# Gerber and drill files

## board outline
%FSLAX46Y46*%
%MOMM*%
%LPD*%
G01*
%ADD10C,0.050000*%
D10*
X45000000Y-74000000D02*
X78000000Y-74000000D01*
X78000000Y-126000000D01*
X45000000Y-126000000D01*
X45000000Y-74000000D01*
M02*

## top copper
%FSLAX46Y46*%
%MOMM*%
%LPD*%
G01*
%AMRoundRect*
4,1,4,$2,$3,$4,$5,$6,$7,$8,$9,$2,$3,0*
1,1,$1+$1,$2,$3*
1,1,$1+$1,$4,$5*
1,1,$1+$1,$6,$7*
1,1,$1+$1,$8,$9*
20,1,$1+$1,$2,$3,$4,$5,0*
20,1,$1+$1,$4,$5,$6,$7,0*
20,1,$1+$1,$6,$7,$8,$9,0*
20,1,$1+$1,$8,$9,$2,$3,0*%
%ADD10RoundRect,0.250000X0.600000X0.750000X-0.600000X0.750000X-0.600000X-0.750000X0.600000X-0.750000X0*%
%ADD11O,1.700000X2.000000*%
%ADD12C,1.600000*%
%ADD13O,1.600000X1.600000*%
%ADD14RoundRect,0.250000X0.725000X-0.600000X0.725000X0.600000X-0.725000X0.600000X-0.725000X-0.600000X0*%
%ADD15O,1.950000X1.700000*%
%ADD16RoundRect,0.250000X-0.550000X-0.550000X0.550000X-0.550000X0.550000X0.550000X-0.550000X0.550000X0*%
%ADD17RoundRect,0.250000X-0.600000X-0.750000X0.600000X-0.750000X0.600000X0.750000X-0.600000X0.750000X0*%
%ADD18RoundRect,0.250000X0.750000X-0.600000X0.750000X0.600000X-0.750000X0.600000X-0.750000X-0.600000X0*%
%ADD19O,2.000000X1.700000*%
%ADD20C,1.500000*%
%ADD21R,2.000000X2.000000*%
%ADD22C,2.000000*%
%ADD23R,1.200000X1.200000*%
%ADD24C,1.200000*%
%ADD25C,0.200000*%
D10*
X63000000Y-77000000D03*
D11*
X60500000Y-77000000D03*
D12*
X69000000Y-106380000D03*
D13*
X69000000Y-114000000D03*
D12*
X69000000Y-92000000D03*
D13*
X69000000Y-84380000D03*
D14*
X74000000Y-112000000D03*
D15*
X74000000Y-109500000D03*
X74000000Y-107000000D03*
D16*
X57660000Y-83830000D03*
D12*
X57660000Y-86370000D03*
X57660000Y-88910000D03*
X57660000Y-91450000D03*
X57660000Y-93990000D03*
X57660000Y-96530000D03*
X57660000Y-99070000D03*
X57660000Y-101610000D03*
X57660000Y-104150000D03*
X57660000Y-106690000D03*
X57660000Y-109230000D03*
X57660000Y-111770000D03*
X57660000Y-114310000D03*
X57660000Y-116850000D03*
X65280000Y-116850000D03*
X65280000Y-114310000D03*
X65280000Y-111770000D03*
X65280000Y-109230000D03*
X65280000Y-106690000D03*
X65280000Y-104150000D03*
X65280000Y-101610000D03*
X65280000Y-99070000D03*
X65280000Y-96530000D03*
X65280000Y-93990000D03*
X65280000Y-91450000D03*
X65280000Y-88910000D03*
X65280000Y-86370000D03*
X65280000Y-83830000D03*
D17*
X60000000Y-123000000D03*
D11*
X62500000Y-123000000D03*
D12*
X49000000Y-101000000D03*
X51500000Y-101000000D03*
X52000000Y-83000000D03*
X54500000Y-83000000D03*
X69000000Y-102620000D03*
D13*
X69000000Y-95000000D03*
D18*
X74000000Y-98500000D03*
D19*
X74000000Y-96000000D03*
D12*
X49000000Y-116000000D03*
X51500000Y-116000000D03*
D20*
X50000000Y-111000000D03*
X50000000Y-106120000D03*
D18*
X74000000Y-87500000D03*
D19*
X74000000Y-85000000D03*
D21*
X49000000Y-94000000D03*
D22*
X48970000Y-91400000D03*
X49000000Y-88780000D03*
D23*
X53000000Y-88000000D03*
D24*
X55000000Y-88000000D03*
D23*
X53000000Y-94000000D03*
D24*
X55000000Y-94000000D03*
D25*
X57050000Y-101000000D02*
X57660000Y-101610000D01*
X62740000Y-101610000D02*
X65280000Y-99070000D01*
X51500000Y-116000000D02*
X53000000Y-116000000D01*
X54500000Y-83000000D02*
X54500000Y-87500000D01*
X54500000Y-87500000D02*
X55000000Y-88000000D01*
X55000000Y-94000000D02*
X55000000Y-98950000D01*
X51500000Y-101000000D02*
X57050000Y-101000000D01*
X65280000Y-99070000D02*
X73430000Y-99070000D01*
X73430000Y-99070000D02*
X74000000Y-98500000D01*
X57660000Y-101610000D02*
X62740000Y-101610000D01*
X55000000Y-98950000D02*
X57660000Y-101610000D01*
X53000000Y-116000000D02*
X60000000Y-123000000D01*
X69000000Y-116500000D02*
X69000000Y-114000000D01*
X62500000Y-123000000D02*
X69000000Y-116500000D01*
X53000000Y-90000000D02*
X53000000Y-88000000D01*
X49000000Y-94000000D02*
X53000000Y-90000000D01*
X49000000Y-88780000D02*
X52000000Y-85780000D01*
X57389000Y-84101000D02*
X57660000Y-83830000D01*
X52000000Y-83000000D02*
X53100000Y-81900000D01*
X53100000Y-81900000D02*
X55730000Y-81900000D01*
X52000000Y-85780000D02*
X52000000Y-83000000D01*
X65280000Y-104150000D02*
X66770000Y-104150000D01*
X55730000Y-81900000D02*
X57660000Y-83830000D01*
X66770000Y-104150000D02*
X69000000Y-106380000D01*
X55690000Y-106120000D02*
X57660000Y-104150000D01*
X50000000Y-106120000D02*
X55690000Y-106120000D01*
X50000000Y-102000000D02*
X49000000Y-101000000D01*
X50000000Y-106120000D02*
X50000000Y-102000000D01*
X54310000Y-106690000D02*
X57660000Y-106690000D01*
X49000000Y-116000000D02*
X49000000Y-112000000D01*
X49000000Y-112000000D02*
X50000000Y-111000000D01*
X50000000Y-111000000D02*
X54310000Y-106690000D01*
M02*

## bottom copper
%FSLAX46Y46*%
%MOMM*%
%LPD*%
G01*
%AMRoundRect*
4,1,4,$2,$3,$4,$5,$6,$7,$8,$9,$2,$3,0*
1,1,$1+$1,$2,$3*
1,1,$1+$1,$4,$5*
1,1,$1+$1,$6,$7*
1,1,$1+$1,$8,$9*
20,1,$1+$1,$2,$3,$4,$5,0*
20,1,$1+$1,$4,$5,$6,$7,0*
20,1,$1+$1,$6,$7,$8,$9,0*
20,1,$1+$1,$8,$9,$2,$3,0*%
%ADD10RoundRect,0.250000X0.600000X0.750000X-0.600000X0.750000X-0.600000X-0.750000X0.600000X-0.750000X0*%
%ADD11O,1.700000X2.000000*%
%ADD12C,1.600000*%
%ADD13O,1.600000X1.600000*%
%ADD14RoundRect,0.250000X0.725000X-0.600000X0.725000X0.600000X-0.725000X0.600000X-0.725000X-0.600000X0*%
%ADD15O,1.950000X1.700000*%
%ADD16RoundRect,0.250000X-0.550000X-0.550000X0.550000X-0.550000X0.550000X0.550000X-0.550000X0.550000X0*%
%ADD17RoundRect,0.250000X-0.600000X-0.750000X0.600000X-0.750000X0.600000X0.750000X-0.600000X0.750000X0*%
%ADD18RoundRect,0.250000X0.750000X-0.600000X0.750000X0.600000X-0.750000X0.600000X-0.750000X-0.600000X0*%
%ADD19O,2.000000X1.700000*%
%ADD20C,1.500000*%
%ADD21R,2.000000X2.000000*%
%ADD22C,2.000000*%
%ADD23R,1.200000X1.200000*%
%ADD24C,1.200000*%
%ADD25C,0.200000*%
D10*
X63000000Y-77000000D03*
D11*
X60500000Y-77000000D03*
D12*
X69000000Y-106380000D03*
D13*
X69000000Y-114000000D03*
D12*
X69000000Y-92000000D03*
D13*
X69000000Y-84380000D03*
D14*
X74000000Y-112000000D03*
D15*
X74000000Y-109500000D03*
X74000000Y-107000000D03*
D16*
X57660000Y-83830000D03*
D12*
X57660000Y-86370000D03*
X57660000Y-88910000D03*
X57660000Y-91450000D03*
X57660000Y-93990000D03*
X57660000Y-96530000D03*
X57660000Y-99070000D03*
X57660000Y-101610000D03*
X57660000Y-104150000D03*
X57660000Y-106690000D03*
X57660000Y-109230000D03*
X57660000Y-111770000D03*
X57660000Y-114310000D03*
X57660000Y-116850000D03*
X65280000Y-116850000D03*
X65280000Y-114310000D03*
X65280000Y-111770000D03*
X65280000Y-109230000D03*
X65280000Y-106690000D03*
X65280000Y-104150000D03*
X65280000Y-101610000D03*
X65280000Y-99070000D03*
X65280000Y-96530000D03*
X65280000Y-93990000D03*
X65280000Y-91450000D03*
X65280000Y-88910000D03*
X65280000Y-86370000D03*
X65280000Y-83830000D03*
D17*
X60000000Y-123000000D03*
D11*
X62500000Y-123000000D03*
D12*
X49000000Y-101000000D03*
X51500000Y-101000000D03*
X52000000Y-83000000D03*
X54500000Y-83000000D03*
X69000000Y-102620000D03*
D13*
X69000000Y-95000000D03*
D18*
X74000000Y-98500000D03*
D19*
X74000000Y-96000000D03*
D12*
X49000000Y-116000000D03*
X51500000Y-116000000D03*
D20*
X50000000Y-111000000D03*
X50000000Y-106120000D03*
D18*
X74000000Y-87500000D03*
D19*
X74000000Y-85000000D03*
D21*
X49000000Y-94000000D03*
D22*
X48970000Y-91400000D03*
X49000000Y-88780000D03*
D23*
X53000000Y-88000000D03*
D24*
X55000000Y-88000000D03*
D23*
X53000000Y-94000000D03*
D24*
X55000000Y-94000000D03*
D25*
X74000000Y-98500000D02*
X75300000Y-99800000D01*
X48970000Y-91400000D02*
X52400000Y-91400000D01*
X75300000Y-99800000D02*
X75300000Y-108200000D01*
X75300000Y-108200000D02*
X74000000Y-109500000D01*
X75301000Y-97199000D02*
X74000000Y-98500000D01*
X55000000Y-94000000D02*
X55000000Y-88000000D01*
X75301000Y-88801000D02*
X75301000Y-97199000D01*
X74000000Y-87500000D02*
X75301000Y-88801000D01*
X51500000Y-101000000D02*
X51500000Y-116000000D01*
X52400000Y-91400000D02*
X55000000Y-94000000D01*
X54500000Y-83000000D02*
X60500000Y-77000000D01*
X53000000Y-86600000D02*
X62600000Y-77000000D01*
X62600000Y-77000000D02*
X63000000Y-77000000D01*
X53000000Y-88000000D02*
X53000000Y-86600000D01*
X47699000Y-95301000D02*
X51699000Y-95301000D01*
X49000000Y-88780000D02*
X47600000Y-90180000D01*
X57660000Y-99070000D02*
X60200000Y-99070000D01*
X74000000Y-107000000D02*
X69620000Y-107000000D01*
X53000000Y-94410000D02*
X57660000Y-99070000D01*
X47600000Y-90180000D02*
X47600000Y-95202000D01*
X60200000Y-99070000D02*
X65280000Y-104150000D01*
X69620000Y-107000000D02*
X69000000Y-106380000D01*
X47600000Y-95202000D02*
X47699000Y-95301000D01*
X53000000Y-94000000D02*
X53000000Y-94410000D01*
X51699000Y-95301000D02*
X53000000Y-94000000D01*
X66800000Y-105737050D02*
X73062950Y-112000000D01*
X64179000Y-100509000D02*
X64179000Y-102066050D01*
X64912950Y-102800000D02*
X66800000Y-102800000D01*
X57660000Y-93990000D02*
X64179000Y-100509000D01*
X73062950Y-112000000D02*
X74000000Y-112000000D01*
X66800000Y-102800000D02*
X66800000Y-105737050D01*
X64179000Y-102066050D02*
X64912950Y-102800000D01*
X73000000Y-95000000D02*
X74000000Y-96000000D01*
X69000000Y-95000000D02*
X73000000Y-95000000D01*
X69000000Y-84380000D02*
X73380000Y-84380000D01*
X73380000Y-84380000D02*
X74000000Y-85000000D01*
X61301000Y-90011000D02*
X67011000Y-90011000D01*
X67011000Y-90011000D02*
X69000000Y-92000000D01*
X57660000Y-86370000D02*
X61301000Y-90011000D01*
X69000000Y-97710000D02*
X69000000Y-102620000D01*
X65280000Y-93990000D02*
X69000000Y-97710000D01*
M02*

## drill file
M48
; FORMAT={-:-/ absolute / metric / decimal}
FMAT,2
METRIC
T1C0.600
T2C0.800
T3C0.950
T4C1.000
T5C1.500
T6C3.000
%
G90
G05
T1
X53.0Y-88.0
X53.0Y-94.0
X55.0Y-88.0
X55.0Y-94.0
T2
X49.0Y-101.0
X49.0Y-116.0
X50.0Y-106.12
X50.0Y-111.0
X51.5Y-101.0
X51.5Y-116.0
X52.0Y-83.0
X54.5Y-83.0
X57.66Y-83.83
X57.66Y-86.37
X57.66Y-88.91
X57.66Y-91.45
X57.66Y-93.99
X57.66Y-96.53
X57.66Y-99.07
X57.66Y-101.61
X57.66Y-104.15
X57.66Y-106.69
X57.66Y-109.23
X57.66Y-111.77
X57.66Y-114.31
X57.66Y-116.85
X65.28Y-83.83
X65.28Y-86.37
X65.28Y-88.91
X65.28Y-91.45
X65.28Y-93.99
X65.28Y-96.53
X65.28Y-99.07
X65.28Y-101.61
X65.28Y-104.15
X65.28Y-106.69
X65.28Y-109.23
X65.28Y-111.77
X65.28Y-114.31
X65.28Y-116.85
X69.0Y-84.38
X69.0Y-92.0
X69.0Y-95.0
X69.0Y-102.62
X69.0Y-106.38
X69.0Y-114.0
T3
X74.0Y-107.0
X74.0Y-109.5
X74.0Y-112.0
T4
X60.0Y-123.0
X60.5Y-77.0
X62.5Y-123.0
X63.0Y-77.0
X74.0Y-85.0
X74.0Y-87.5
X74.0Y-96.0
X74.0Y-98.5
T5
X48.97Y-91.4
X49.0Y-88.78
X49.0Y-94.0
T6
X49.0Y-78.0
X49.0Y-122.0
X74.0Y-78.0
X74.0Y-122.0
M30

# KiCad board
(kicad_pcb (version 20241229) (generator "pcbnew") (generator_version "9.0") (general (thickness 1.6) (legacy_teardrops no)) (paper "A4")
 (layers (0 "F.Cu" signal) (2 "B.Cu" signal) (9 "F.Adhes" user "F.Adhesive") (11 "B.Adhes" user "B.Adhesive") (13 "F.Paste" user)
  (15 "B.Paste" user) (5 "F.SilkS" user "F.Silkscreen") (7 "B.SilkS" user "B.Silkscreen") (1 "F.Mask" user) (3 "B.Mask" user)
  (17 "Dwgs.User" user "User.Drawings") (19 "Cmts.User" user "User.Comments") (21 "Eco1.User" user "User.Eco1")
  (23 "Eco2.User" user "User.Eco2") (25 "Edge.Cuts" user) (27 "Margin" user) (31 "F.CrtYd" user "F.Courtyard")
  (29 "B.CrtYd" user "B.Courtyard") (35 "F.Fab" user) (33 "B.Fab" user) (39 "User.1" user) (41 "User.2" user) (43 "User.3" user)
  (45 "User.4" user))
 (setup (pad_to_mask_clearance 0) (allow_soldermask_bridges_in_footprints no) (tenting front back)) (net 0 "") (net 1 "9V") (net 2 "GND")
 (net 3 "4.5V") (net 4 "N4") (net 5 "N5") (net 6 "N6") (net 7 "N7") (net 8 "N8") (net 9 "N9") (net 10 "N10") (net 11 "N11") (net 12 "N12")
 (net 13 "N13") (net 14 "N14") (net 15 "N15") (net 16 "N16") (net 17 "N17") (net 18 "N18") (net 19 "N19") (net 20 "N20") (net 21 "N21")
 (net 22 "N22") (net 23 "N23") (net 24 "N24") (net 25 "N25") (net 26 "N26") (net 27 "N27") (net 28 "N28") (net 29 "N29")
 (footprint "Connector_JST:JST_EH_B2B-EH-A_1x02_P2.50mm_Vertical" (layer "F.Cu") (at 63 77 180)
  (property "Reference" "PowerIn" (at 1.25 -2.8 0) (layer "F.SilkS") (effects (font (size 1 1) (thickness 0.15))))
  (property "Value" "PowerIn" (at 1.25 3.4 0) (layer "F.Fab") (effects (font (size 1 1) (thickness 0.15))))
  (pad "1" thru_hole roundrect (at 0 0 180) (size 1.7 2) (drill 1) (layers "*.Cu" "*.Mask") (remove_unused_layers no)
   (roundrect_rratio 0.147059) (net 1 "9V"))
  (pad "2" thru_hole oval (at 2.5 0 180) (size 1.7 2) (drill 1) (layers "*.Cu" "*.Mask") (remove_unused_layers no) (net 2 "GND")))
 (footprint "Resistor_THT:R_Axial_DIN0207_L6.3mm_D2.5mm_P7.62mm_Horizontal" (layer "F.Cu") (at 69 106.38 -90)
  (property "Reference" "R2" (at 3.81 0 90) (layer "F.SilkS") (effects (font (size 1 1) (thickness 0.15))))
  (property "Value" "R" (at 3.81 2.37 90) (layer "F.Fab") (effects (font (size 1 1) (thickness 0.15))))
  (pad "1" thru_hole circle (at 0 0 270) (size 1.6 1.6) (drill 0.8) (layers "*.Cu" "*.Mask") (remove_unused_layers no) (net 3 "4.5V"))
  (pad "2" thru_hole oval (at 7.62 0 270) (size 1.6 1.6) (drill 0.8) (layers "*.Cu" "*.Mask") (remove_unused_layers no) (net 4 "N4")))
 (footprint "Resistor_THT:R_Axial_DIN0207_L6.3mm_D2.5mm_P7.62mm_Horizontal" (layer "F.Cu") (at 69 92 90)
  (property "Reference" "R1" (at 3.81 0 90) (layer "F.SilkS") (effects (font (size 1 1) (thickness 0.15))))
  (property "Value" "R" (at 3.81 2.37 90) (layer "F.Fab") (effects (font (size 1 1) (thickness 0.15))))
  (pad "1" thru_hole circle (at 0 0 90) (size 1.6 1.6) (drill 0.8) (layers "*.Cu" "*.Mask") (remove_unused_layers no) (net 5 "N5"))
  (pad "2" thru_hole oval (at 7.62 0 90) (size 1.6 1.6) (drill 0.8) (layers "*.Cu" "*.Mask") (remove_unused_layers no) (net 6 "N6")))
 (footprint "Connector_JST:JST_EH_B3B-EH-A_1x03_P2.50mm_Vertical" (layer "F.Cu") (at 74 112 90)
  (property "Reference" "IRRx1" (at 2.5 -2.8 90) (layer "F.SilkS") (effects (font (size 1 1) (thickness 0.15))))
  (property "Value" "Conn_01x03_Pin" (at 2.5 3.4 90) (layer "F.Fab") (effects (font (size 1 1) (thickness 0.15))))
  (pad "1" thru_hole roundrect (at 0 0 90) (size 1.7 1.95) (drill 0.95) (layers "*.Cu" "*.Mask") (remove_unused_layers no)
   (roundrect_rratio 0.147059) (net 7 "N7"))
  (pad "2" thru_hole oval (at 2.5 0 90) (size 1.7 1.95) (drill 0.95) (layers "*.Cu" "*.Mask") (remove_unused_layers no) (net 2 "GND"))
  (pad "3" thru_hole oval (at 5 0 90) (size 1.7 1.95) (drill 0.95) (layers "*.Cu" "*.Mask") (remove_unused_layers no) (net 3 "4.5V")))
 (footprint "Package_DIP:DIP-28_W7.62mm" (layer "F.Cu") (at 57.66 83.83)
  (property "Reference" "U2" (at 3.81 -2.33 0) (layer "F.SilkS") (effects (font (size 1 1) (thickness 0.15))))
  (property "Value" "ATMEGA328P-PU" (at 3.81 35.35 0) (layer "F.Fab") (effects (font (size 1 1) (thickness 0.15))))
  (pad "1" thru_hole roundrect (at 0 0) (size 1.6 1.6) (drill 0.8) (layers "*.Cu" "*.Mask") (remove_unused_layers no)
   (roundrect_rratio 0.15625) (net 3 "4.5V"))
  (pad "2" thru_hole circle (at 0 2.54) (size 1.6 1.6) (drill 0.8) (layers "*.Cu" "*.Mask") (remove_unused_layers no) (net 5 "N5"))
  (pad "3" thru_hole circle (at 0 5.08) (size 1.6 1.6) (drill 0.8) (layers "*.Cu" "*.Mask") (remove_unused_layers no) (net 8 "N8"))
  (pad "4" thru_hole circle (at 0 7.62) (size 1.6 1.6) (drill 0.8) (layers "*.Cu" "*.Mask") (remove_unused_layers no) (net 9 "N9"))
  (pad "5" thru_hole circle (at 0 10.16) (size 1.6 1.6) (drill 0.8) (layers "*.Cu" "*.Mask") (remove_unused_layers no) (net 7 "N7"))
  (pad "6" thru_hole circle (at 0 12.7) (size 1.6 1.6) (drill 0.8) (layers "*.Cu" "*.Mask") (remove_unused_layers no) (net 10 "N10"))
  (pad "7" thru_hole circle (at 0 15.24) (size 1.6 1.6) (drill 0.8) (layers "*.Cu" "*.Mask") (remove_unused_layers no) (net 3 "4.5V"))
  (pad "8" thru_hole circle (at 0 17.78) (size 1.6 1.6) (drill 0.8) (layers "*.Cu" "*.Mask") (remove_unused_layers no) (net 2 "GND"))
  (pad "9" thru_hole circle (at 0 20.32) (size 1.6 1.6) (drill 0.8) (layers "*.Cu" "*.Mask") (remove_unused_layers no) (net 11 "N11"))
  (pad "10" thru_hole circle (at 0 22.86) (size 1.6 1.6) (drill 0.8) (layers "*.Cu" "*.Mask") (remove_unused_layers no) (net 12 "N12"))
  (pad "11" thru_hole circle (at 0 25.4) (size 1.6 1.6) (drill 0.8) (layers "*.Cu" "*.Mask") (remove_unused_layers no) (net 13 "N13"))
  (pad "12" thru_hole circle (at 0 27.94) (size 1.6 1.6) (drill 0.8) (layers "*.Cu" "*.Mask") (remove_unused_layers no) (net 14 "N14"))
  (pad "13" thru_hole circle (at 0 30.48) (size 1.6 1.6) (drill 0.8) (layers "*.Cu" "*.Mask") (remove_unused_layers no) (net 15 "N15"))
  (pad "14" thru_hole circle (at 0 33.02) (size 1.6 1.6) (drill 0.8) (layers "*.Cu" "*.Mask") (remove_unused_layers no) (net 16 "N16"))
  (pad "15" thru_hole circle (at 7.62 33.02) (size 1.6 1.6) (drill 0.8) (layers "*.Cu" "*.Mask") (remove_unused_layers no) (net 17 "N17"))
  (pad "16" thru_hole circle (at 7.62 30.48) (size 1.6 1.6) (drill 0.8) (layers "*.Cu" "*.Mask") (remove_unused_layers no) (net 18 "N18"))
  (pad "17" thru_hole circle (at 7.62 27.94) (size 1.6 1.6) (drill 0.8) (layers "*.Cu" "*.Mask") (remove_unused_layers no) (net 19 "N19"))
  (pad "18" thru_hole circle (at 7.62 25.4) (size 1.6 1.6) (drill 0.8) (layers "*.Cu" "*.Mask") (remove_unused_layers no) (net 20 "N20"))
  (pad "19" thru_hole circle (at 7.62 22.86) (size 1.6 1.6) (drill 0.8) (layers "*.Cu" "*.Mask") (remove_unused_layers no) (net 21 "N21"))
  (pad "20" thru_hole circle (at 7.62 20.32) (size 1.6 1.6) (drill 0.8) (layers "*.Cu" "*.Mask") (remove_unused_layers no) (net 3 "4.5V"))
  (pad "21" thru_hole circle (at 7.62 17.78) (size 1.6 1.6) (drill 0.8) (layers "*.Cu" "*.Mask") (remove_unused_layers no) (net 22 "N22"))
  (pad "22" thru_hole circle (at 7.62 15.24) (size 1.6 1.6) (drill 0.8) (layers "*.Cu" "*.Mask") (remove_unused_layers no) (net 2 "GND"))
  (pad "23" thru_hole circle (at 7.62 12.7) (size 1.6 1.6) (drill 0.8) (layers "*.Cu" "*.Mask") (remove_unused_layers no) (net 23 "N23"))
  (pad "24" thru_hole circle (at 7.62 10.16) (size 1.6 1.6) (drill 0.8) (layers "*.Cu" "*.Mask") (remove_unused_layers no) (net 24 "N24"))
  (pad "25" thru_hole circle (at 7.62 7.62) (size 1.6 1.6) (drill 0.8) (layers "*.Cu" "*.Mask") (remove_unused_layers no) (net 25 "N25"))
  (pad "26" thru_hole circle (at 7.62 5.08) (size 1.6 1.6) (drill 0.8) (layers "*.Cu" "*.Mask") (remove_unused_layers no) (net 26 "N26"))
  (pad "27" thru_hole circle (at 7.62 2.54) (size 1.6 1.6) (drill 0.8) (layers "*.Cu" "*.Mask") (remove_unused_layers no) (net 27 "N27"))
  (pad "28" thru_hole circle (at 7.62 0) (size 1.6 1.6) (drill 0.8) (layers "*.Cu" "*.Mask") (remove_unused_layers no) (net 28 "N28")))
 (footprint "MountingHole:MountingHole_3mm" (layer "F.Cu") (at 49 122)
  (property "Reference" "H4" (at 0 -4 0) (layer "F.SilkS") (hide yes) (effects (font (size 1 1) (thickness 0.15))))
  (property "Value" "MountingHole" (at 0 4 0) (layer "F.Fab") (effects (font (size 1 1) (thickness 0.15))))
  (pad "" np_thru_hole circle (at 0 0) (size 3 3) (drill 3) (layers "*.Cu" "*.Mask")))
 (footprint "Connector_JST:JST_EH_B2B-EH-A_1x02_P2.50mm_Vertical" (layer "F.Cu") (at 60 123)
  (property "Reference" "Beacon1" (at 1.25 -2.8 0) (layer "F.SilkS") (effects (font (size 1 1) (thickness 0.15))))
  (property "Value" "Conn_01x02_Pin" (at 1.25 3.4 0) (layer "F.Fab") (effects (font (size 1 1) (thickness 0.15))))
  (pad "1" thru_hole roundrect (at 0 0) (size 1.7 2) (drill 1) (layers "*.Cu" "*.Mask") (remove_unused_layers no)
   (roundrect_rratio 0.147059) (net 2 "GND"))
  (pad "2" thru_hole oval (at 2.5 0) (size 1.7 2) (drill 1) (layers "*.Cu" "*.Mask") (remove_unused_layers no) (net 4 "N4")))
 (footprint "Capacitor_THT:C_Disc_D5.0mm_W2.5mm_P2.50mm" (layer "F.Cu") (at 49 101)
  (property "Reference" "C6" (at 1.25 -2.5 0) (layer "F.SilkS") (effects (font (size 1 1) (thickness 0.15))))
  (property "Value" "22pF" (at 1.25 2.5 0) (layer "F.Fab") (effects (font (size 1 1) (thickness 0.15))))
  (pad "1" thru_hole circle (at 0 0) (size 1.6 1.6) (drill 0.8) (layers "*.Cu" "*.Mask") (remove_unused_layers no) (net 11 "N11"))
  (pad "2" thru_hole circle (at 2.5 0) (size 1.6 1.6) (drill 0.8) (layers "*.Cu" "*.Mask") (remove_unused_layers no) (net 2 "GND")))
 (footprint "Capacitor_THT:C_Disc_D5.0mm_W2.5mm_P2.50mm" (layer "F.Cu") (at 52 83)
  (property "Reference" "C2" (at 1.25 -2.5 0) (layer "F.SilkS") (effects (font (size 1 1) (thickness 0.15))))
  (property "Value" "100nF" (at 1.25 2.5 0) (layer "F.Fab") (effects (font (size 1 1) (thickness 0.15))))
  (pad "1" thru_hole circle (at 0 0) (size 1.6 1.6) (drill 0.8) (layers "*.Cu" "*.Mask") (remove_unused_layers no) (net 3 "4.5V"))
  (pad "2" thru_hole circle (at 2.5 0) (size 1.6 1.6) (drill 0.8) (layers "*.Cu" "*.Mask") (remove_unused_layers no) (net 2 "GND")))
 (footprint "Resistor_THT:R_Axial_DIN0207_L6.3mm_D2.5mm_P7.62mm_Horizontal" (layer "F.Cu") (at 69 102.62 90)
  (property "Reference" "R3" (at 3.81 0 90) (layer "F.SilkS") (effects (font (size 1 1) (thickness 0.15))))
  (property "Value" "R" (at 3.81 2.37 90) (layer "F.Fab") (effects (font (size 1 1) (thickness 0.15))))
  (pad "1" thru_hole circle (at 0 0 90) (size 1.6 1.6) (drill 0.8) (layers "*.Cu" "*.Mask") (remove_unused_layers no) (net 24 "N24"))
  (pad "2" thru_hole oval (at 7.62 0 90) (size 1.6 1.6) (drill 0.8) (layers "*.Cu" "*.Mask") (remove_unused_layers no) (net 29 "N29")))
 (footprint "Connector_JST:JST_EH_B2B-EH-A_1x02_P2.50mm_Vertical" (layer "F.Cu") (at 74 98.5 90)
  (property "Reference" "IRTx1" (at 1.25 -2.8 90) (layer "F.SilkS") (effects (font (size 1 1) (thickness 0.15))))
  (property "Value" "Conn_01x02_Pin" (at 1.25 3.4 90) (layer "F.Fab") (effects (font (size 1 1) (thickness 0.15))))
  (pad "1" thru_hole roundrect (at 0 0 90) (size 1.7 2) (drill 1) (layers "*.Cu" "*.Mask") (remove_unused_layers no)
   (roundrect_rratio 0.147059) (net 2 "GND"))
  (pad "2" thru_hole oval (at 2.5 0 90) (size 1.7 2) (drill 1) (layers "*.Cu" "*.Mask") (remove_unused_layers no) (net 29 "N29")))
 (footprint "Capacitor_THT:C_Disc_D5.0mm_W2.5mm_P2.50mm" (layer "F.Cu") (at 49 116)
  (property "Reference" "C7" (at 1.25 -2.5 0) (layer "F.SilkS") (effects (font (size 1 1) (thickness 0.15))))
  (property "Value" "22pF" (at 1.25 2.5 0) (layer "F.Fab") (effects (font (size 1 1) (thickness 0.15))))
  (pad "1" thru_hole circle (at 0 0) (size 1.6 1.6) (drill 0.8) (layers "*.Cu" "*.Mask") (remove_unused_layers no) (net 12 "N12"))
  (pad "2" thru_hole circle (at 2.5 0) (size 1.6 1.6) (drill 0.8) (layers "*.Cu" "*.Mask") (remove_unused_layers no) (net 2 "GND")))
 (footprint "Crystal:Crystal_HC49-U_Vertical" (layer "F.Cu") (at 50 111 90)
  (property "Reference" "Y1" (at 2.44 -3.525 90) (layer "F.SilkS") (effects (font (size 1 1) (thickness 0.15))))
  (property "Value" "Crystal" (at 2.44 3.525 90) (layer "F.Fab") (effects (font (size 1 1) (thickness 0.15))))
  (pad "1" thru_hole circle (at 0 0 90) (size 1.5 1.5) (drill 0.8) (layers "*.Cu" "*.Mask") (remove_unused_layers no) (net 12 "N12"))
  (pad "2" thru_hole circle (at 4.88 0 90) (size 1.5 1.5) (drill 0.8) (layers "*.Cu" "*.Mask") (remove_unused_layers no) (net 11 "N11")))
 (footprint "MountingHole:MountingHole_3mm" (layer "F.Cu") (at 74 122)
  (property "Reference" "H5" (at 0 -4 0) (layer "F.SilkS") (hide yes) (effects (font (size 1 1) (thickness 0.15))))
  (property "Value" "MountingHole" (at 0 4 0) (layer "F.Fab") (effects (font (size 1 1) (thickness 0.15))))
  (pad "" np_thru_hole circle (at 0 0) (size 3 3) (drill 3) (layers "*.Cu" "*.Mask")))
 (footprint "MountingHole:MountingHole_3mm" (layer "F.Cu") (at 49 78)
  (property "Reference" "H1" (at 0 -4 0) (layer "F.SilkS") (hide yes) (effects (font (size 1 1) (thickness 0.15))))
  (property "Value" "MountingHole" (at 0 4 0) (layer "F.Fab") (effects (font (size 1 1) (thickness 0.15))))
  (pad "" np_thru_hole circle (at 0 0) (size 3 3) (drill 3) (layers "*.Cu" "*.Mask")))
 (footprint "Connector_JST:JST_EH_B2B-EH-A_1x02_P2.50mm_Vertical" (layer "F.Cu") (at 74 87.5 90)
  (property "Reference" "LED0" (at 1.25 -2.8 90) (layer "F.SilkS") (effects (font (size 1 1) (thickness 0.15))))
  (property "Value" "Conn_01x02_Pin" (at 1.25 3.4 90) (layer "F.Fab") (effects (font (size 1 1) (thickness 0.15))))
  (pad "1" thru_hole roundrect (at 0 0 90) (size 1.7 2) (drill 1) (layers "*.Cu" "*.Mask") (remove_unused_layers no)
   (roundrect_rratio 0.147059) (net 2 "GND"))
  (pad "2" thru_hole oval (at 2.5 0 90) (size 1.7 2) (drill 1) (layers "*.Cu" "*.Mask") (remove_unused_layers no) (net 6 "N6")))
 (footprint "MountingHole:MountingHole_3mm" (layer "F.Cu") (at 74 78)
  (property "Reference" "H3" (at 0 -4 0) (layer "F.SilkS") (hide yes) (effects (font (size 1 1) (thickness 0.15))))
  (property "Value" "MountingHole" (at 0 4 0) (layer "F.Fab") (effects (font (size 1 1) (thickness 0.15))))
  (pad "" np_thru_hole circle (at 0 0) (size 3 3) (drill 3) (layers "*.Cu" "*.Mask")))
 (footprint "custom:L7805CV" (layer "F.Cu") (at 48.08 95.01 90)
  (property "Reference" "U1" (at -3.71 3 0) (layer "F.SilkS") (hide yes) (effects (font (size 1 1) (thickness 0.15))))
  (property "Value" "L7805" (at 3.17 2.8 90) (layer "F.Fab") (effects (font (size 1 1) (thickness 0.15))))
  (pad "1" thru_hole rect (at 1.01 0.92 90) (size 2 2) (drill 1.5) (layers "*.Cu" "*.Mask") (remove_unused_layers no) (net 1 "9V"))
  (pad "2" thru_hole circle (at 3.61 0.89 90) (size 2 2) (drill 1.5) (layers "*.Cu" "*.Mask") (remove_unused_layers no) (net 2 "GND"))
  (pad "3" thru_hole circle (at 6.23 0.92 90) (size 2 2) (drill 1.5) (layers "*.Cu" "*.Mask") (remove_unused_layers no) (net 3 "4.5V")))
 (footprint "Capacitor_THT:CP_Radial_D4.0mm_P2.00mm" (layer "F.Cu") (at 53 88)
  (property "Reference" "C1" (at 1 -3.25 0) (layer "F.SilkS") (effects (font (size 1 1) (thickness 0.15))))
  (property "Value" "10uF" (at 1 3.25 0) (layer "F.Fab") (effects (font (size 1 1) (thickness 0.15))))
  (pad "1" thru_hole rect (at 0 0) (size 1.2 1.2) (drill 0.6) (layers "*.Cu" "*.Mask") (remove_unused_layers no) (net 1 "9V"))
  (pad "2" thru_hole circle (at 2 0) (size 1.2 1.2) (drill 0.6) (layers "*.Cu" "*.Mask") (remove_unused_layers no) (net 2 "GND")))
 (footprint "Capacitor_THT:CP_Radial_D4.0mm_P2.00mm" (layer "F.Cu") (at 53 94)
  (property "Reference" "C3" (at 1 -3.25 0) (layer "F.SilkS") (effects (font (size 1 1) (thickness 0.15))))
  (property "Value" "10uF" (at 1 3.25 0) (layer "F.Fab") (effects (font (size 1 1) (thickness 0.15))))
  (pad "1" thru_hole rect (at 0 0) (size 1.2 1.2) (drill 0.6) (layers "*.Cu" "*.Mask") (remove_unused_layers no) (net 3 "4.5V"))
  (pad "2" thru_hole circle (at 2 0) (size 1.2 1.2) (drill 0.6) (layers "*.Cu" "*.Mask") (remove_unused_layers no) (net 2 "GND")))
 (gr_rect (start 45 74) (end 78 126) (stroke (width 0.05) (type default)) (fill no) (layer "Edge.Cuts"))
 (segment (start 57.05 101) (end 57.66 101.61) (width 0.2) (layer "F.Cu") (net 2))
 (segment (start 62.74 101.61) (end 65.28 99.07) (width 0.2) (layer "F.Cu") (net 2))
 (segment (start 51.5 116) (end 53 116) (width 0.2) (layer "F.Cu") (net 2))
 (segment (start 54.5 83) (end 54.5 87.5) (width 0.2) (layer "F.Cu") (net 2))
 (segment (start 54.5 87.5) (end 55 88) (width 0.2) (layer "F.Cu") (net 2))
 (segment (start 55 94) (end 55 98.95) (width 0.2) (layer "F.Cu") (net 2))
 (segment (start 51.5 101) (end 57.05 101) (width 0.2) (layer "F.Cu") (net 2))
 (segment (start 65.28 99.07) (end 73.43 99.07) (width 0.2) (layer "F.Cu") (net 2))
 (segment (start 73.43 99.07) (end 74 98.5) (width 0.2) (layer "F.Cu") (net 2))
 (segment (start 57.66 101.61) (end 62.74 101.61) (width 0.2) (layer "F.Cu") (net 2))
 (segment (start 55 98.95) (end 57.66 101.61) (width 0.2) (layer "F.Cu") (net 2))
 (segment (start 53 116) (end 60 123) (width 0.2) (layer "F.Cu") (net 2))
 (segment (start 74 98.5) (end 75.3 99.8) (width 0.2) (layer "B.Cu") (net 2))
 (segment (start 48.97 91.4) (end 52.4 91.4) (width 0.2) (layer "B.Cu") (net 2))
 (segment (start 75.3 99.8) (end 75.3 108.2) (width 0.2) (layer "B.Cu") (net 2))
 (segment (start 75.3 108.2) (end 74 109.5) (width 0.2) (layer "B.Cu") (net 2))
 (segment (start 75.301 97.199) (end 74 98.5) (width 0.2) (layer "B.Cu") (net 2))
 (segment (start 55 94) (end 55 88) (width 0.2) (layer "B.Cu") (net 2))
 (segment (start 75.301 88.801) (end 75.301 97.199) (width 0.2) (layer "B.Cu") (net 2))
 (segment (start 74 87.5) (end 75.301 88.801) (width 0.2) (layer "B.Cu") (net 2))
 (segment (start 51.5 101) (end 51.5 116) (width 0.2) (layer "B.Cu") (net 2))
 (segment (start 52.4 91.4) (end 55 94) (width 0.2) (layer "B.Cu") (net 2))
 (segment (start 54.5 83) (end 60.5 77) (width 0.2) (layer "B.Cu") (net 2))
 (segment (start 69 116.5) (end 69 114) (width 0.2) (layer "F.Cu") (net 4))
 (segment (start 62.5 123) (end 69 116.5) (width 0.2) (layer "F.Cu") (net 4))
 (segment (start 53 90) (end 53 88) (width 0.2) (layer "F.Cu") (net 1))
 (segment (start 49 94) (end 53 90) (width 0.2) (layer "F.Cu") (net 1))
 (segment (start 53 86.6) (end 62.6 77) (width 0.2) (layer "B.Cu") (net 1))
 (segment (start 62.6 77) (end 63 77) (width 0.2) (layer "B.Cu") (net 1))
 (segment (start 53 88) (end 53 86.6) (width 0.2) (layer "B.Cu") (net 1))
 (segment (start 49 88.78) (end 52 85.78) (width 0.2) (layer "F.Cu") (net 3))
 (segment (start 57.389 84.101) (end 57.66 83.83) (width 0.2) (layer "F.Cu") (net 3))
 (segment (start 52 83) (end 53.1 81.9) (width 0.2) (layer "F.Cu") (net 3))
 (segment (start 53.1 81.9) (end 55.73 81.9) (width 0.2) (layer "F.Cu") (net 3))
 (segment (start 52 85.78) (end 52 83) (width 0.2) (layer "F.Cu") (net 3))
 (segment (start 65.28 104.15) (end 66.77 104.15) (width 0.2) (layer "F.Cu") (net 3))
 (segment (start 55.73 81.9) (end 57.66 83.83) (width 0.2) (layer "F.Cu") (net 3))
 (segment (start 66.77 104.15) (end 69 106.38) (width 0.2) (layer "F.Cu") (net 3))
 (segment (start 47.699 95.301) (end 51.699 95.301) (width 0.2) (layer "B.Cu") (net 3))
 (segment (start 49 88.78) (end 47.6 90.18) (width 0.2) (layer "B.Cu") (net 3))
 (segment (start 57.66 99.07) (end 60.2 99.07) (width 0.2) (layer "B.Cu") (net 3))
 (segment (start 74 107) (end 69.62 107) (width 0.2) (layer "B.Cu") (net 3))
 (segment (start 53 94.41) (end 57.66 99.07) (width 0.2) (layer "B.Cu") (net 3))
 (segment (start 47.6 90.18) (end 47.6 95.202) (width 0.2) (layer "B.Cu") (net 3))
 (segment (start 60.2 99.07) (end 65.28 104.15) (width 0.2) (layer "B.Cu") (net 3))
 (segment (start 69.62 107) (end 69 106.38) (width 0.2) (layer "B.Cu") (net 3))
 (segment (start 47.6 95.202) (end 47.699 95.301) (width 0.2) (layer "B.Cu") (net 3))
 (segment (start 53 94) (end 53 94.41) (width 0.2) (layer "B.Cu") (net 3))
 (segment (start 51.699 95.301) (end 53 94) (width 0.2) (layer "B.Cu") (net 3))
 (segment (start 55.69 106.12) (end 57.66 104.15) (width 0.2) (layer "F.Cu") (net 11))
 (segment (start 50 106.12) (end 55.69 106.12) (width 0.2) (layer "F.Cu") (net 11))
 (segment (start 50 102) (end 49 101) (width 0.2) (layer "F.Cu") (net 11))
 (segment (start 50 106.12) (end 50 102) (width 0.2) (layer "F.Cu") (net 11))
 (segment (start 54.31 106.69) (end 57.66 106.69) (width 0.2) (layer "F.Cu") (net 12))
 (segment (start 49 116) (end 49 112) (width 0.2) (layer "F.Cu") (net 12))
 (segment (start 49 112) (end 50 111) (width 0.2) (layer "F.Cu") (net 12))
 (segment (start 50 111) (end 54.31 106.69) (width 0.2) (layer "F.Cu") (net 12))
 (segment (start 66.8 105.73705) (end 73.06295 112) (width 0.2) (layer "B.Cu") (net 7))
 (segment (start 64.179 100.509) (end 64.179 102.06605) (width 0.2) (layer "B.Cu") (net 7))
 (segment (start 64.91295 102.8) (end 66.8 102.8) (width 0.2) (layer "B.Cu") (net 7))
 (segment (start 57.66 93.99) (end 64.179 100.509) (width 0.2) (layer "B.Cu") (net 7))
 (segment (start 73.06295 112) (end 74 112) (width 0.2) (layer "B.Cu") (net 7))
 (segment (start 66.8 102.8) (end 66.8 105.73705) (width 0.2) (layer "B.Cu") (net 7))
 (segment (start 64.179 102.06605) (end 64.91295 102.8) (width 0.2) (layer "B.Cu") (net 7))
 (segment (start 73 95) (end 74 96) (width 0.2) (layer "B.Cu") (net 29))
 (segment (start 69 95) (end 73 95) (width 0.2) (layer "B.Cu") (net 29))
 (segment (start 69 84.38) (end 73.38 84.38) (width 0.2) (layer "B.Cu") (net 6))
 (segment (start 73.38 84.38) (end 74 85) (width 0.2) (layer "B.Cu") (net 6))
 (segment (start 61.301 90.011) (end 67.011 90.011) (width 0.2) (layer "B.Cu") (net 5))
 (segment (start 67.011 90.011) (end 69 92) (width 0.2) (layer "B.Cu") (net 5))
 (segment (start 57.66 86.37) (end 61.301 90.011) (width 0.2) (layer "B.Cu") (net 5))
 (segment (start 69 97.71) (end 69 102.62) (width 0.2) (layer "B.Cu") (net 24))
 (segment (start 65.28 93.99) (end 69 97.71) (width 0.2) (layer "B.Cu") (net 24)))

